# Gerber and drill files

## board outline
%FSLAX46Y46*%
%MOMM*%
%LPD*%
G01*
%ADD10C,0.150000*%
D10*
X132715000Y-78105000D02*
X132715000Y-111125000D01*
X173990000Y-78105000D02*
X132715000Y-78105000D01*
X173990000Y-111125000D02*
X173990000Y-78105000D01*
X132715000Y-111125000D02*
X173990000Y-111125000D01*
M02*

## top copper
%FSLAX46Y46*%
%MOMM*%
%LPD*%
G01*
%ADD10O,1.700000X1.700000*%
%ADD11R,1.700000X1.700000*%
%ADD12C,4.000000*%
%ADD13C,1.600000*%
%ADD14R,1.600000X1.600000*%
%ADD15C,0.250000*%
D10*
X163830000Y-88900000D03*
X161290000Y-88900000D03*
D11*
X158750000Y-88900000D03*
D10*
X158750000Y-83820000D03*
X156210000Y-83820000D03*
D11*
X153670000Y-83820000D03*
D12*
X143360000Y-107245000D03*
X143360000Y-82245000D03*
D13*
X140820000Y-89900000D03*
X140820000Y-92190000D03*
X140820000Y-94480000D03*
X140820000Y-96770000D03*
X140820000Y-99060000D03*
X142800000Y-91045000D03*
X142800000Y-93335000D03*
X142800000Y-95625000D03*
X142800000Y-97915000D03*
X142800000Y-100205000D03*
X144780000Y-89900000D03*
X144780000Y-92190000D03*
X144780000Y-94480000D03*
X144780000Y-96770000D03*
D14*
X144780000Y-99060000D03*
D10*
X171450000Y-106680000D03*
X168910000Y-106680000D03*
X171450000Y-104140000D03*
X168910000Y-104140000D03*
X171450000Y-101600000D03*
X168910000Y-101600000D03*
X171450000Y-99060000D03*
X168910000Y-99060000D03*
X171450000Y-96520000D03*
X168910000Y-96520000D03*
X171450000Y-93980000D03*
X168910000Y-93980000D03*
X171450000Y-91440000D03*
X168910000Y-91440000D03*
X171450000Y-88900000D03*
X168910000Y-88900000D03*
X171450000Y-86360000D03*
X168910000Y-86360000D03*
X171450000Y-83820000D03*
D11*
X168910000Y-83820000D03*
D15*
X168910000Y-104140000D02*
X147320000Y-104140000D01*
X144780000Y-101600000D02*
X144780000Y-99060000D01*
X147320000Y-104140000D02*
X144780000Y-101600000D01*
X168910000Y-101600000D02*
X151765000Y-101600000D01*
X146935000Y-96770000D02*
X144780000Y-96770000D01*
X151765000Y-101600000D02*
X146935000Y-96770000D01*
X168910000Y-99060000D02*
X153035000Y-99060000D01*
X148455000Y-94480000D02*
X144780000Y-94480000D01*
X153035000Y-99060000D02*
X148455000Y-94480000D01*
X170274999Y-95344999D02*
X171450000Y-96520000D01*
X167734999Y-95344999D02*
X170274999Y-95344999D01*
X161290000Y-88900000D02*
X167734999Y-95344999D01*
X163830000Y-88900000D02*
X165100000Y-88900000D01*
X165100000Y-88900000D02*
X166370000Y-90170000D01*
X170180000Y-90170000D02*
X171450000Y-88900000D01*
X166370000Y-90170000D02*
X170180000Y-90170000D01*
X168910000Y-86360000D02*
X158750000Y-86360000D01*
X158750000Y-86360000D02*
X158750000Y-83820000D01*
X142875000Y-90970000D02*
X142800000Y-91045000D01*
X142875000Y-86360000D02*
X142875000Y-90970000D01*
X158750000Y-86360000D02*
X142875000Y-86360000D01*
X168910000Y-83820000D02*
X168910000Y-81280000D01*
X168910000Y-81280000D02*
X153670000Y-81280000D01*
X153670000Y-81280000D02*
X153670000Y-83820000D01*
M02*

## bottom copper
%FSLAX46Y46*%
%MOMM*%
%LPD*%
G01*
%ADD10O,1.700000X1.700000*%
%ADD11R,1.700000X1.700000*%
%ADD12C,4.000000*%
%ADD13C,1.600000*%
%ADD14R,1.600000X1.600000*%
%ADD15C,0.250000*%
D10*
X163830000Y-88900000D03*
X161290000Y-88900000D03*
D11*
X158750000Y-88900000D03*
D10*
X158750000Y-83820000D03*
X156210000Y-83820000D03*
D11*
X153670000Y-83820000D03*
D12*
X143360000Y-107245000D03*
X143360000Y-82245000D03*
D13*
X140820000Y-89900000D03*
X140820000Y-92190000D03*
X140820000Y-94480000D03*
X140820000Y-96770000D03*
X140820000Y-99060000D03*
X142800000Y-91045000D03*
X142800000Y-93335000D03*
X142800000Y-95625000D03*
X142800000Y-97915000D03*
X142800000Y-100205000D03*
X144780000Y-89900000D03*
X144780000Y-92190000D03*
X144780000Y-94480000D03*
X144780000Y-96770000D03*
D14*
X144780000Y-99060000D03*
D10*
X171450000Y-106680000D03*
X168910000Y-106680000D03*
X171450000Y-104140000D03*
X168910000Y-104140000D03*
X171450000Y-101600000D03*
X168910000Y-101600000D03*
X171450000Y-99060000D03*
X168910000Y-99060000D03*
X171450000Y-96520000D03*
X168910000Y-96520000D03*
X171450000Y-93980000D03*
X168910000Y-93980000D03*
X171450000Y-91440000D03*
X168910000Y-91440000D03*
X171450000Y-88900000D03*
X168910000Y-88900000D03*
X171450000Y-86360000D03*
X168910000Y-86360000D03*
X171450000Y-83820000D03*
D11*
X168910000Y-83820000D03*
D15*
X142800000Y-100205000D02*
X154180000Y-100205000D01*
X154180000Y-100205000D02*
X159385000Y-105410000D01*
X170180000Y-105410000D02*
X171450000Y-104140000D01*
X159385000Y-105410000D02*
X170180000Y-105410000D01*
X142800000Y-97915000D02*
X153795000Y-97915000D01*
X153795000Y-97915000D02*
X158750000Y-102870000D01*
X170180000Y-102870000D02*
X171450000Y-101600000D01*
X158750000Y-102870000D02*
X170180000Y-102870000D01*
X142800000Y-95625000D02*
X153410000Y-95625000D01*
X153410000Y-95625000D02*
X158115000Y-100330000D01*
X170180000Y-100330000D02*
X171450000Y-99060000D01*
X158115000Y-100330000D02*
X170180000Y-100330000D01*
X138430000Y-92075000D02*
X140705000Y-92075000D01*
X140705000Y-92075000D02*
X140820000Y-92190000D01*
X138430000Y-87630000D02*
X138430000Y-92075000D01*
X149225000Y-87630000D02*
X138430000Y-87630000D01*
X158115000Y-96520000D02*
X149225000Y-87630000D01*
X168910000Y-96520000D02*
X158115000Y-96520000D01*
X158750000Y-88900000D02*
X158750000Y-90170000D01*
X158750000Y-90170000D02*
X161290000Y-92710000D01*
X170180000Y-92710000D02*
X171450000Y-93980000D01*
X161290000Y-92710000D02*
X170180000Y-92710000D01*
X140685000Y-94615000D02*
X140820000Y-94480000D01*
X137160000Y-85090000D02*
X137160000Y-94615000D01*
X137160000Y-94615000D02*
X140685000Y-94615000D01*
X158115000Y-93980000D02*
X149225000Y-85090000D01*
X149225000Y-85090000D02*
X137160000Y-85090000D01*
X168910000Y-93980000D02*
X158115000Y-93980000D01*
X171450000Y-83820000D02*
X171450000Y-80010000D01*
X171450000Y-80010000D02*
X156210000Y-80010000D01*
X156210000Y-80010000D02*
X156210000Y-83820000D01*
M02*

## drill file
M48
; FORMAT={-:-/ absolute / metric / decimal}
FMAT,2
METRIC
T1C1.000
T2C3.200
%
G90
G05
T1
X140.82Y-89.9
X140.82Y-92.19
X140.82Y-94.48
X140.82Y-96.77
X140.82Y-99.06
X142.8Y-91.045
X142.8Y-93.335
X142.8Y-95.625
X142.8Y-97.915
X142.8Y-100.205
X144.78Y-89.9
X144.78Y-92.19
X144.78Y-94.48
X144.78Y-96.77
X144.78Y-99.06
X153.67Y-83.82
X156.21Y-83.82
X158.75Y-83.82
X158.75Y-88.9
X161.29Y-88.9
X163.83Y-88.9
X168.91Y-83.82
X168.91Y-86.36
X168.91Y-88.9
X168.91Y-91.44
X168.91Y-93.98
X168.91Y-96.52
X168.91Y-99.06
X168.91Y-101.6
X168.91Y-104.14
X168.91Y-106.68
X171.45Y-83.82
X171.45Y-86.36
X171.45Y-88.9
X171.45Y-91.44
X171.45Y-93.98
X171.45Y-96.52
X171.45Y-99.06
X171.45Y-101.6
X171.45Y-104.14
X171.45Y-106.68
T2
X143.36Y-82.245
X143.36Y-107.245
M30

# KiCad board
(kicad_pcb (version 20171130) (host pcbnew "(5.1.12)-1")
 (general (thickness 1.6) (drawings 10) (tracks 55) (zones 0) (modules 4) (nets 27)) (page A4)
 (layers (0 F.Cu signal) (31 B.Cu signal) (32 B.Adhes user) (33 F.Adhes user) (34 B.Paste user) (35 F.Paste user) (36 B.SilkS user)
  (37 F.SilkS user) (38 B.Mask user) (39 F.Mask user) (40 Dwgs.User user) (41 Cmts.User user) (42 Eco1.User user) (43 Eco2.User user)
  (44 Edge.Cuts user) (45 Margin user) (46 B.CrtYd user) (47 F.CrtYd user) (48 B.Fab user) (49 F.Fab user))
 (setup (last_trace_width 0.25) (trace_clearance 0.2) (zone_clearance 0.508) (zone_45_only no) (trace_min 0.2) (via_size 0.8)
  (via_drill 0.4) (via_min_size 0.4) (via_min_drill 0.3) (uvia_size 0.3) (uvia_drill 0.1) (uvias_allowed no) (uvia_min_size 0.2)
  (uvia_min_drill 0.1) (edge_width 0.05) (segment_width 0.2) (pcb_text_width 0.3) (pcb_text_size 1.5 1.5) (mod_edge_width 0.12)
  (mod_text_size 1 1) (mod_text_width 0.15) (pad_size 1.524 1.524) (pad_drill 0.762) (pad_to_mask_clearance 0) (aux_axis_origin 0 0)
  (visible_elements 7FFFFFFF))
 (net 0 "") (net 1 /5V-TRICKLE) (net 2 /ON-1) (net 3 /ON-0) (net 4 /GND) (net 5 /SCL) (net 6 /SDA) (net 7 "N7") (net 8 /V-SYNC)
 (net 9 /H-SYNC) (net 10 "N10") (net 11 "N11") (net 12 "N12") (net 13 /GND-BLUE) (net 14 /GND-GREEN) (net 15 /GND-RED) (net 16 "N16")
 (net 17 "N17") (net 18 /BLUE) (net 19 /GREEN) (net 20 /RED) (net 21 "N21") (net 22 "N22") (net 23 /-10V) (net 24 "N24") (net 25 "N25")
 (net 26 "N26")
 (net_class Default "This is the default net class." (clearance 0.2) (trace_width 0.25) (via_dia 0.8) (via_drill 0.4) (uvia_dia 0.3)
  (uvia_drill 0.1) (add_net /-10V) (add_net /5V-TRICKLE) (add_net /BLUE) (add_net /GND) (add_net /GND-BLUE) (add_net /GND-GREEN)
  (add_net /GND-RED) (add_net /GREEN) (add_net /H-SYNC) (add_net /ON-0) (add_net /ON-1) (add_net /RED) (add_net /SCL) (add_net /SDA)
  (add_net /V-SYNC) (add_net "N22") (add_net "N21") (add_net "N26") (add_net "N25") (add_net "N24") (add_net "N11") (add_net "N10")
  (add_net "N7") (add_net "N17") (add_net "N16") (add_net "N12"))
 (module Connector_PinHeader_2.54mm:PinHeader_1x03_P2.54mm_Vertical (layer F.Cu) (at 158.75 88.9 90)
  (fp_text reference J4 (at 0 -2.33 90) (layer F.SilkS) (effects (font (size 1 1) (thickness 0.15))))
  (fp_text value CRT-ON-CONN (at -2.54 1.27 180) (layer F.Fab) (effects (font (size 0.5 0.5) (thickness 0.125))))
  (pad 3 thru_hole oval (at 0 5.08 90) (size 1.7 1.7) (drill 1) (layers *.Cu *.Mask) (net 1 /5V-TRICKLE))
  (pad 2 thru_hole oval (at 0 2.54 90) (size 1.7 1.7) (drill 1) (layers *.Cu *.Mask) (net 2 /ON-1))
  (pad 1 thru_hole rect (at 0 0 90) (size 1.7 1.7) (drill 1) (layers *.Cu *.Mask) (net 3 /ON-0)))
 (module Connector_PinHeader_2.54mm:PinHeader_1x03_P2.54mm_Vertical (layer F.Cu) (at 153.67 83.82 90)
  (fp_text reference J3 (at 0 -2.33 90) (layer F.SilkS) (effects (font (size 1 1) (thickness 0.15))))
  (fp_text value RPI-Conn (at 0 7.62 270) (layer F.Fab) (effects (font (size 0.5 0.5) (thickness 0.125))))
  (pad 3 thru_hole oval (at 0 5.08 90) (size 1.7 1.7) (drill 1) (layers *.Cu *.Mask) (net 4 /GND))
  (pad 2 thru_hole oval (at 0 2.54 90) (size 1.7 1.7) (drill 1) (layers *.Cu *.Mask) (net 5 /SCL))
  (pad 1 thru_hole rect (at 0 0 90) (size 1.7 1.7) (drill 1) (layers *.Cu *.Mask) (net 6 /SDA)))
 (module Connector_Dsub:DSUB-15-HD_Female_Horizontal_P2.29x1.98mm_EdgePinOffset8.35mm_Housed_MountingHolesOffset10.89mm (layer F.Cu)
  (at 144.78 99.06 270)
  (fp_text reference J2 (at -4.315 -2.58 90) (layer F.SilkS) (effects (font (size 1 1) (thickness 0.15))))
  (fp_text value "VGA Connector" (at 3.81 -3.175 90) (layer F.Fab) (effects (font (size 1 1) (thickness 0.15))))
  (pad 0 thru_hole circle (at 8.185 1.42 270) (size 4 4) (drill 3.2) (layers *.Cu *.Mask))
  (pad 0 thru_hole circle (at -16.815 1.42 270) (size 4 4) (drill 3.2) (layers *.Cu *.Mask))
  (pad 15 thru_hole circle (at -9.16 3.96 270) (size 1.6 1.6) (drill 1) (layers *.Cu *.Mask) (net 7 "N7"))
  (pad 14 thru_hole circle (at -6.87 3.96 270) (size 1.6 1.6) (drill 1) (layers *.Cu *.Mask) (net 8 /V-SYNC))
  (pad 13 thru_hole circle (at -4.58 3.96 270) (size 1.6 1.6) (drill 1) (layers *.Cu *.Mask) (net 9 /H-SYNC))
  (pad 12 thru_hole circle (at -2.29 3.96 270) (size 1.6 1.6) (drill 1) (layers *.Cu *.Mask) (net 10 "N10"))
  (pad 11 thru_hole circle (at 0 3.96 270) (size 1.6 1.6) (drill 1) (layers *.Cu *.Mask) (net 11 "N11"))
  (pad 10 thru_hole circle (at -8.015 1.98 270) (size 1.6 1.6) (drill 1) (layers *.Cu *.Mask) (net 4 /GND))
  (pad 9 thru_hole circle (at -5.725 1.98 270) (size 1.6 1.6) (drill 1) (layers *.Cu *.Mask) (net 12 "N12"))
  (pad 8 thru_hole circle (at -3.435 1.98 270) (size 1.6 1.6) (drill 1) (layers *.Cu *.Mask) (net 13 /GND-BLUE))
  (pad 7 thru_hole circle (at -1.145 1.98 270) (size 1.6 1.6) (drill 1) (layers *.Cu *.Mask) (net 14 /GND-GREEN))
  (pad 6 thru_hole circle (at 1.145 1.98 270) (size 1.6 1.6) (drill 1) (layers *.Cu *.Mask) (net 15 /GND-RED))
  (pad 5 thru_hole circle (at -9.16 0 270) (size 1.6 1.6) (drill 1) (layers *.Cu *.Mask) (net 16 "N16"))
  (pad 4 thru_hole circle (at -6.87 0 270) (size 1.6 1.6) (drill 1) (layers *.Cu *.Mask) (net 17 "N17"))
  (pad 3 thru_hole circle (at -4.58 0 270) (size 1.6 1.6) (drill 1) (layers *.Cu *.Mask) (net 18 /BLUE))
  (pad 2 thru_hole circle (at -2.29 0 270) (size 1.6 1.6) (drill 1) (layers *.Cu *.Mask) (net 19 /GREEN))
  (pad 1 thru_hole rect (at 0 0 270) (size 1.6 1.6) (drill 1) (layers *.Cu *.Mask) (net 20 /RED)))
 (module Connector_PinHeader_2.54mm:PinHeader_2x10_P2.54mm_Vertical (layer F.Cu) (at 168.91 83.82)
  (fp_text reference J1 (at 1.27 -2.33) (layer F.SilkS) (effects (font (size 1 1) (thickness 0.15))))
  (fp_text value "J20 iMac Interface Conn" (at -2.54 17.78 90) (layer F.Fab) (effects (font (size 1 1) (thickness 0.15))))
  (pad 20 thru_hole oval (at 2.54 22.86) (size 1.7 1.7) (drill 1) (layers *.Cu *.Mask) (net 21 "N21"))
  (pad 19 thru_hole oval (at 0 22.86) (size 1.7 1.7) (drill 1) (layers *.Cu *.Mask) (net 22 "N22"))
  (pad 18 thru_hole oval (at 2.54 20.32) (size 1.7 1.7) (drill 1) (layers *.Cu *.Mask) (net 15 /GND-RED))
  (pad 17 thru_hole oval (at 0 20.32) (size 1.7 1.7) (drill 1) (layers *.Cu *.Mask) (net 20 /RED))
  (pad 16 thru_hole oval (at 2.54 17.78) (size 1.7 1.7) (drill 1) (layers *.Cu *.Mask) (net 14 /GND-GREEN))
  (pad 15 thru_hole oval (at 0 17.78) (size 1.7 1.7) (drill 1) (layers *.Cu *.Mask) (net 19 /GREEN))
  (pad 14 thru_hole oval (at 2.54 15.24) (size 1.7 1.7) (drill 1) (layers *.Cu *.Mask) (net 13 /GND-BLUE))
  (pad 13 thru_hole oval (at 0 15.24) (size 1.7 1.7) (drill 1) (layers *.Cu *.Mask) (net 18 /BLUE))
  (pad 12 thru_hole oval (at 2.54 12.7) (size 1.7 1.7) (drill 1) (layers *.Cu *.Mask) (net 2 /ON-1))
  (pad 11 thru_hole oval (at 0 12.7) (size 1.7 1.7) (drill 1) (layers *.Cu *.Mask) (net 8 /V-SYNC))
  (pad 10 thru_hole oval (at 2.54 10.16) (size 1.7 1.7) (drill 1) (layers *.Cu *.Mask) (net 3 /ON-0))
  (pad 9 thru_hole oval (at 0 10.16) (size 1.7 1.7) (drill 1) (layers *.Cu *.Mask) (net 9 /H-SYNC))
  (pad 8 thru_hole oval (at 2.54 7.62) (size 1.7 1.7) (drill 1) (layers *.Cu *.Mask) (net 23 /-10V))
  (pad 7 thru_hole oval (at 0 7.62) (size 1.7 1.7) (drill 1) (layers *.Cu *.Mask) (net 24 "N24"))
  (pad 6 thru_hole oval (at 2.54 5.08) (size 1.7 1.7) (drill 1) (layers *.Cu *.Mask) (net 1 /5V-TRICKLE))
  (pad 5 thru_hole oval (at 0 5.08) (size 1.7 1.7) (drill 1) (layers *.Cu *.Mask) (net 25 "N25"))
  (pad 4 thru_hole oval (at 2.54 2.54) (size 1.7 1.7) (drill 1) (layers *.Cu *.Mask) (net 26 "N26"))
  (pad 3 thru_hole oval (at 0 2.54) (size 1.7 1.7) (drill 1) (layers *.Cu *.Mask) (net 4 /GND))
  (pad 2 thru_hole oval (at 2.54 0) (size 1.7 1.7) (drill 1) (layers *.Cu *.Mask) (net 5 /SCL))
  (pad 1 thru_hole rect (at 0 0) (size 1.7 1.7) (drill 1) (layers *.Cu *.Mask) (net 6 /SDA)))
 (gr_line (start 132.715 78.105) (end 132.715 111.125) (layer Edge.Cuts) (width 0.15))
 (gr_line (start 173.99 78.105) (end 132.715 78.105) (layer Edge.Cuts) (width 0.15))
 (gr_line (start 173.99 111.125) (end 173.99 78.105) (layer Edge.Cuts) (width 0.15))
 (gr_line (start 132.715 111.125) (end 173.99 111.125) (layer Edge.Cuts) (width 0.15))
 (segment (start 142.8 100.205) (end 154.18 100.205) (width 0.25) (layer B.Cu) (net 15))
 (segment (start 154.18 100.205) (end 159.385 105.41) (width 0.25) (layer B.Cu) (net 15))
 (segment (start 170.18 105.41) (end 171.45 104.14) (width 0.25) (layer B.Cu) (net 15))
 (segment (start 159.385 105.41) (end 170.18 105.41) (width 0.25) (layer B.Cu) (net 15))
 (segment (start 168.91 104.14) (end 147.32 104.14) (width 0.25) (layer F.Cu) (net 20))
 (segment (start 144.78 101.6) (end 144.78 99.06) (width 0.25) (layer F.Cu) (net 20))
 (segment (start 147.32 104.14) (end 144.78 101.6) (width 0.25) (layer F.Cu) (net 20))
 (segment (start 142.8 97.915) (end 153.795 97.915) (width 0.25) (layer B.Cu) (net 14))
 (segment (start 153.795 97.915) (end 158.75 102.87) (width 0.25) (layer B.Cu) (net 14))
 (segment (start 170.18 102.87) (end 171.45 101.6) (width 0.25) (layer B.Cu) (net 14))
 (segment (start 158.75 102.87) (end 170.18 102.87) (width 0.25) (layer B.Cu) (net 14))
 (segment (start 168.91 101.6) (end 151.765 101.6) (width 0.25) (layer F.Cu) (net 19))
 (segment (start 146.935 96.77) (end 144.78 96.77) (width 0.25) (layer F.Cu) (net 19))
 (segment (start 151.765 101.6) (end 146.935 96.77) (width 0.25) (layer F.Cu) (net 19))
 (segment (start 142.8 95.625) (end 153.41 95.625) (width 0.25) (layer B.Cu) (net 13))
 (segment (start 153.41 95.625) (end 158.115 100.33) (width 0.25) (layer B.Cu) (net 13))
 (segment (start 170.18 100.33) (end 171.45 99.06) (width 0.25) (layer B.Cu) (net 13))
 (segment (start 158.115 100.33) (end 170.18 100.33) (width 0.25) (layer B.Cu) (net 13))
 (segment (start 168.91 99.06) (end 153.035 99.06) (width 0.25) (layer F.Cu) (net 18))
 (segment (start 148.455 94.48) (end 144.78 94.48) (width 0.25) (layer F.Cu) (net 18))
 (segment (start 153.035 99.06) (end 148.455 94.48) (width 0.25) (layer F.Cu) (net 18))
 (segment (start 170.274999 95.344999) (end 171.45 96.52) (width 0.25) (layer F.Cu) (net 2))
 (segment (start 167.734999 95.344999) (end 170.274999 95.344999) (width 0.25) (layer F.Cu) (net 2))
 (segment (start 161.29 88.9) (end 167.734999 95.344999) (width 0.25) (layer F.Cu) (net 2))
 (segment (start 138.43 92.075) (end 140.705 92.075) (width 0.25) (layer B.Cu) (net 8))
 (segment (start 140.705 92.075) (end 140.82 92.19) (width 0.25) (layer B.Cu) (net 8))
 (segment (start 138.43 87.63) (end 138.43 92.075) (width 0.25) (layer B.Cu) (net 8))
 (segment (start 149.225 87.63) (end 138.43 87.63) (width 0.25) (layer B.Cu) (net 8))
 (segment (start 158.115 96.52) (end 149.225 87.63) (width 0.25) (layer B.Cu) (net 8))
 (segment (start 168.91 96.52) (end 158.115 96.52) (width 0.25) (layer B.Cu) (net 8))
 (segment (start 158.75 88.9) (end 158.75 90.17) (width 0.25) (layer B.Cu) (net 3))
 (segment (start 158.75 90.17) (end 161.29 92.71) (width 0.25) (layer B.Cu) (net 3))
 (segment (start 170.18 92.71) (end 171.45 93.98) (width 0.25) (layer B.Cu) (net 3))
 (segment (start 161.29 92.71) (end 170.18 92.71) (width 0.25) (layer B.Cu) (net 3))
 (segment (start 140.685 94.615) (end 140.82 94.48) (width 0.25) (layer B.Cu) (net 9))
 (segment (start 137.16 85.09) (end 137.16 94.615) (width 0.25) (layer B.Cu) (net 9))
 (segment (start 137.16 94.615) (end 140.685 94.615) (width 0.25) (layer B.Cu) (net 9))
 (segment (start 158.115 93.98) (end 149.225 85.09) (width 0.25) (layer B.Cu) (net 9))
 (segment (start 149.225 85.09) (end 137.16 85.09) (width 0.25) (layer B.Cu) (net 9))
 (segment (start 168.91 93.98) (end 158.115 93.98) (width 0.25) (layer B.Cu) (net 9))
 (segment (start 163.83 88.9) (end 165.1 88.9) (width 0.25) (layer F.Cu) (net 1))
 (segment (start 165.1 88.9) (end 166.37 90.17) (width 0.25) (layer F.Cu) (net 1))
 (segment (start 170.18 90.17) (end 171.45 88.9) (width 0.25) (layer F.Cu) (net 1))
 (segment (start 166.37 90.17) (end 170.18 90.17) (width 0.25) (layer F.Cu) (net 1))
 (segment (start 168.91 86.36) (end 158.75 86.36) (width 0.25) (layer F.Cu) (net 4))
 (segment (start 158.75 86.36) (end 158.75 83.82) (width 0.25) (layer F.Cu) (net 4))
 (segment (start 142.875 90.97) (end 142.8 91.045) (width 0.25) (layer F.Cu) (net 4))
 (segment (start 142.875 86.36) (end 142.875 90.97) (width 0.25) (layer F.Cu) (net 4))
 (segment (start 158.75 86.36) (end 142.875 86.36) (width 0.25) (layer F.Cu) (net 4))
 (segment (start 171.45 83.82) (end 171.45 80.01) (width 0.25) (layer B.Cu) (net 5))
 (segment (start 171.45 80.01) (end 156.21 80.01) (width 0.25) (layer B.Cu) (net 5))
 (segment (start 156.21 80.01) (end 156.21 83.82) (width 0.25) (layer B.Cu) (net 5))
 (segment (start 168.91 83.82) (end 168.91 81.28) (width 0.25) (layer F.Cu) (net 6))
 (segment (start 168.91 81.28) (end 153.67 81.28) (width 0.25) (layer F.Cu) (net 6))
 (segment (start 153.67 81.28) (end 153.67 83.82) (width 0.25) (layer F.Cu) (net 6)))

